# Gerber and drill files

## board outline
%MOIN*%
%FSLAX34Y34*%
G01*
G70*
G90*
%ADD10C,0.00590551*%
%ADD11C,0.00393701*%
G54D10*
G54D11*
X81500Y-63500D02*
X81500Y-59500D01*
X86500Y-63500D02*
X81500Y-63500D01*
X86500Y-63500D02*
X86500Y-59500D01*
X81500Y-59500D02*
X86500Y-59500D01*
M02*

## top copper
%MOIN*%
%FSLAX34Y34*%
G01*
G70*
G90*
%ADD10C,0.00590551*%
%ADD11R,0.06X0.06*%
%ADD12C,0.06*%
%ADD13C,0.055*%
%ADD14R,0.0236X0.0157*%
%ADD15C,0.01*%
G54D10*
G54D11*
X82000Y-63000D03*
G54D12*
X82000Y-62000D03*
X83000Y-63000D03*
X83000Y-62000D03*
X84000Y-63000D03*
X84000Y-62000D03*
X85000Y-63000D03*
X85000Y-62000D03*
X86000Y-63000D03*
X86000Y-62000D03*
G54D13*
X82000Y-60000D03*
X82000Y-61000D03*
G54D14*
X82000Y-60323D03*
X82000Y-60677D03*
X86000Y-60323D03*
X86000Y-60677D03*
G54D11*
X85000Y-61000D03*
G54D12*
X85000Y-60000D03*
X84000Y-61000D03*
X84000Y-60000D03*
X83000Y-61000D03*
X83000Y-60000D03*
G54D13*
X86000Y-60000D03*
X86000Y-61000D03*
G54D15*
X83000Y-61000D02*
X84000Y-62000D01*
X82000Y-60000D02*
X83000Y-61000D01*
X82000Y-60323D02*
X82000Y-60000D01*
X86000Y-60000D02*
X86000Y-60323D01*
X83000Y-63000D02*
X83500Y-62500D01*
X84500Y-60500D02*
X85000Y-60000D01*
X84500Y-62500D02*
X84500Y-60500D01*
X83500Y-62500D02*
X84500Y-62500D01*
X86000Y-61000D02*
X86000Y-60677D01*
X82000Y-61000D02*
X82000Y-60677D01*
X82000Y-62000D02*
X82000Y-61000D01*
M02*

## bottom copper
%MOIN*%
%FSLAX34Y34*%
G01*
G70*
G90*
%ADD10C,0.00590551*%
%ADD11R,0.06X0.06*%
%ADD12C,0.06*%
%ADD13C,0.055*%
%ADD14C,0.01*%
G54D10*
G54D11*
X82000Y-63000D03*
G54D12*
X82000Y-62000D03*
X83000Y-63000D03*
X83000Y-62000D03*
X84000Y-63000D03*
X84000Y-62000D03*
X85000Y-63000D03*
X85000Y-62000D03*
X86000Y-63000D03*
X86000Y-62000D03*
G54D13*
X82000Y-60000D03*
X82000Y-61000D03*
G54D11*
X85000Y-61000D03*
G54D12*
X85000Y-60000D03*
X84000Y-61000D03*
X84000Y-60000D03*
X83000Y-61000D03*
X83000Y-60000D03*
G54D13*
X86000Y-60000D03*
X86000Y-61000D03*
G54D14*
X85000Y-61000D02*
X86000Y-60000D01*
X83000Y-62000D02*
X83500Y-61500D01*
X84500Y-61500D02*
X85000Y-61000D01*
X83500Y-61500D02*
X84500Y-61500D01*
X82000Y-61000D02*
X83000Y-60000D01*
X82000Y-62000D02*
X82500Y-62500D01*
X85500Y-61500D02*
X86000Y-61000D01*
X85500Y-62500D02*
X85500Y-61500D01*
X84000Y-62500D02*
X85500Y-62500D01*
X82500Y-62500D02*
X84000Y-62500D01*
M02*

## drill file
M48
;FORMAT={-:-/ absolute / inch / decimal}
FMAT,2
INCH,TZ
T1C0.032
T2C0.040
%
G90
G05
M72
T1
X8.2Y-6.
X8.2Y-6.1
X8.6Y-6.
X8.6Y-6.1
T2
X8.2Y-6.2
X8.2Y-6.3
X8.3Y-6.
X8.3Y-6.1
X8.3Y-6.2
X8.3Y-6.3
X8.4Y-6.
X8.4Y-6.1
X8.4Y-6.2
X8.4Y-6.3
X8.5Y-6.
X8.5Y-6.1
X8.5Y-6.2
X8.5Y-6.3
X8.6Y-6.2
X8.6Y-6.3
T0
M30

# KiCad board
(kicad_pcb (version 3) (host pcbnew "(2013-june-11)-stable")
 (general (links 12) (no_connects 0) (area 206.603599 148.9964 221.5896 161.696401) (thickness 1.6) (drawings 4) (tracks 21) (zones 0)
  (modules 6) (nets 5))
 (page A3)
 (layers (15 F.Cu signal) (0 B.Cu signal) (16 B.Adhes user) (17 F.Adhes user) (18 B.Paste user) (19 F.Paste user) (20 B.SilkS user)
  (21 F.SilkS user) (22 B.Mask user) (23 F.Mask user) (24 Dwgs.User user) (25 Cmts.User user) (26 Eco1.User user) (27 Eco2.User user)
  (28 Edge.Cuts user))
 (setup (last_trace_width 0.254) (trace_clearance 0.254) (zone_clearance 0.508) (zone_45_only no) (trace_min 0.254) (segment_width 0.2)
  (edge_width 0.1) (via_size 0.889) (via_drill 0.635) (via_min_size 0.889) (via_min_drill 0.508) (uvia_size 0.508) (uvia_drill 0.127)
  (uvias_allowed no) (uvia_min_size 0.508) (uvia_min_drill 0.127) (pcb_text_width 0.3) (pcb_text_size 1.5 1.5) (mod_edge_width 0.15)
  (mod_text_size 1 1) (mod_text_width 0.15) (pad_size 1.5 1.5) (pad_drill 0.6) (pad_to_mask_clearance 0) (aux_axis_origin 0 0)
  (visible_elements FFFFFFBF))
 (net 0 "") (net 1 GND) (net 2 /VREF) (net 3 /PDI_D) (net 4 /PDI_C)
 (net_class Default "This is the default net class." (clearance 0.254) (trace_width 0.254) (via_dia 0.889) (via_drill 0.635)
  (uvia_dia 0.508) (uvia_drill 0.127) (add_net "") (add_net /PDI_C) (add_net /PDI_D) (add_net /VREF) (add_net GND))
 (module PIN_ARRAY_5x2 (layer F.Cu) (at 213.36 158.75)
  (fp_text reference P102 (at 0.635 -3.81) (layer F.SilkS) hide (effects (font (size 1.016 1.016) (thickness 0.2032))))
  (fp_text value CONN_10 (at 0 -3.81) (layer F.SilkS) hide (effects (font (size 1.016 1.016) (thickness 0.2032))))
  (pad 1 thru_hole rect (at -5.08 1.27) (size 1.524 1.524) (drill 1.016) (layers *.Cu *.Mask F.SilkS))
  (pad 2 thru_hole circle (at -5.08 -1.27) (size 1.524 1.524) (drill 1.016) (layers *.Cu *.Mask F.SilkS) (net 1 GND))
  (pad 3 thru_hole circle (at -2.54 1.27) (size 1.524 1.524) (drill 1.016) (layers *.Cu *.Mask F.SilkS) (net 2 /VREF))
  (pad 4 thru_hole circle (at -2.54 -1.27) (size 1.524 1.524) (drill 1.016) (layers *.Cu *.Mask F.SilkS) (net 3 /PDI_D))
  (pad 5 thru_hole circle (at 0 1.27) (size 1.524 1.524) (drill 1.016) (layers *.Cu *.Mask F.SilkS))
  (pad 6 thru_hole circle (at 0 -1.27) (size 1.524 1.524) (drill 1.016) (layers *.Cu *.Mask F.SilkS) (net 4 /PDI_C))
  (pad 7 thru_hole circle (at 2.54 1.27) (size 1.524 1.524) (drill 1.016) (layers *.Cu *.Mask F.SilkS))
  (pad 8 thru_hole circle (at 2.54 -1.27) (size 1.524 1.524) (drill 1.016) (layers *.Cu *.Mask F.SilkS))
  (pad 9 thru_hole circle (at 5.08 1.27) (size 1.524 1.524) (drill 1.016) (layers *.Cu *.Mask F.SilkS))
  (pad 10 thru_hole circle (at 5.08 -1.27) (size 1.524 1.524) (drill 1.016) (layers *.Cu *.Mask F.SilkS)))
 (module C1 (layer F.Cu) (at 208.28 153.67 270)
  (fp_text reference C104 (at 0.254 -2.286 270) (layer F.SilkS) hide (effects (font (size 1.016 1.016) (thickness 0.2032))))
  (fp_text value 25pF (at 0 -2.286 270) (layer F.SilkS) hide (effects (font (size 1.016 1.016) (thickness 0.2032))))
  (pad 1 thru_hole circle (at -1.27 0 270) (size 1.397 1.397) (drill 0.8128) (layers *.Cu *.Mask F.SilkS) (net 4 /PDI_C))
  (pad 2 thru_hole circle (at 1.27 0 270) (size 1.397 1.397) (drill 0.8128) (layers *.Cu *.Mask F.SilkS) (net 1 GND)))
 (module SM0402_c (layer F.Cu) (at 208.28 153.67 270)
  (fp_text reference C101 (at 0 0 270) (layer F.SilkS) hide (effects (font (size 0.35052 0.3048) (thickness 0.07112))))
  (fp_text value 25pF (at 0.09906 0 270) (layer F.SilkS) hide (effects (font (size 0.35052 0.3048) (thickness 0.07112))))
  (pad 1 smd rect (at -0.44958 0 270) (size 0.39878 0.59944) (layers F.Cu F.Paste F.Mask) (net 4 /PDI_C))
  (pad 2 smd rect (at 0.44958 0 270) (size 0.39878 0.59944) (layers F.Cu F.Paste F.Mask) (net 1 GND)))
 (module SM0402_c (layer F.Cu) (at 218.44 153.67 270)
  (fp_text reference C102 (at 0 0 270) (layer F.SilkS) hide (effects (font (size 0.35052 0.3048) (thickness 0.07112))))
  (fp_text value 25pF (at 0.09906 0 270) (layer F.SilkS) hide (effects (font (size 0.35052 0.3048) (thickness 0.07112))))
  (pad 1 smd rect (at -0.44958 0 270) (size 0.39878 0.59944) (layers F.Cu F.Paste F.Mask) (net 3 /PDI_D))
  (pad 2 smd rect (at 0.44958 0 270) (size 0.39878 0.59944) (layers F.Cu F.Paste F.Mask) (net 1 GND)))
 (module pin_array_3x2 (layer B.Cu) (at 213.36 153.67 180)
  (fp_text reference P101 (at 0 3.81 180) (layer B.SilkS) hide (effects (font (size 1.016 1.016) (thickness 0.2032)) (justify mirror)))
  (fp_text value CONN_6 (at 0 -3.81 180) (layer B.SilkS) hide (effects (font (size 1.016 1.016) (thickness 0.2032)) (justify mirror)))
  (pad 1 thru_hole rect (at -2.54 -1.27 180) (size 1.524 1.524) (drill 1.016) (layers *.Cu *.Mask B.SilkS) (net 3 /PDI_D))
  (pad 2 thru_hole circle (at -2.54 1.27 180) (size 1.524 1.524) (drill 1.016) (layers *.Cu *.Mask B.SilkS) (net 2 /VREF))
  (pad 3 thru_hole circle (at 0 -1.27 180) (size 1.524 1.524) (drill 1.016) (layers *.Cu *.Mask B.SilkS))
  (pad 4 thru_hole circle (at 0 1.27 180) (size 1.524 1.524) (drill 1.016) (layers *.Cu *.Mask B.SilkS))
  (pad 5 thru_hole circle (at 2.54 -1.27 180) (size 1.524 1.524) (drill 1.016) (layers *.Cu *.Mask B.SilkS) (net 4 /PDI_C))
  (pad 6 thru_hole circle (at 2.54 1.27 180) (size 1.524 1.524) (drill 1.016) (layers *.Cu *.Mask B.SilkS) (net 1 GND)))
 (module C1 (layer F.Cu) (at 218.44 153.67 270)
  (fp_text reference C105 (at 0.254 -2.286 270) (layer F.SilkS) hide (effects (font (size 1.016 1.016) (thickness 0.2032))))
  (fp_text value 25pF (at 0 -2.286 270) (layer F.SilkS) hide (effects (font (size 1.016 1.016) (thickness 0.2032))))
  (pad 1 thru_hole circle (at -1.27 0 270) (size 1.397 1.397) (drill 0.8128) (layers *.Cu *.Mask F.SilkS) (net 3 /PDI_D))
  (pad 2 thru_hole circle (at 1.27 0 270) (size 1.397 1.397) (drill 0.8128) (layers *.Cu *.Mask F.SilkS) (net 1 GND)))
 (gr_line (start 207.01 161.29) (end 207.01 151.13) (angle 90) (layer Edge.Cuts) (width 0.1))
 (gr_line (start 219.71 161.29) (end 207.01 161.29) (angle 90) (layer Edge.Cuts) (width 0.1))
 (gr_line (start 219.71 161.29) (end 219.71 151.13) (angle 90) (layer Edge.Cuts) (width 0.1))
 (gr_line (start 207.01 151.13) (end 219.71 151.13) (angle 90) (layer Edge.Cuts) (width 0.1))
 (segment (start 210.82 154.94) (end 213.36 157.48) (width 0.254) (layer F.Cu) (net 4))
 (segment (start 208.28 152.4) (end 210.82 154.94) (width 0.254) (layer F.Cu) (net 4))
 (segment (start 208.28 153.22042) (end 208.28 152.4) (width 0.254) (layer F.Cu) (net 4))
 (segment (start 215.9 154.94) (end 218.44 152.4) (width 0.254) (layer B.Cu) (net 3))
 (segment (start 210.82 157.48) (end 212.09 156.21) (width 0.254) (layer B.Cu) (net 3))
 (segment (start 214.63 156.21) (end 215.9 154.94) (width 0.254) (layer B.Cu) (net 3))
 (segment (start 212.09 156.21) (end 214.63 156.21) (width 0.254) (layer B.Cu) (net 3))
 (segment (start 218.44 152.4) (end 218.44 153.22042) (width 0.254) (layer F.Cu) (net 3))
 (segment (start 210.82 160.02) (end 212.09 158.75) (width 0.254) (layer F.Cu) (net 2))
 (segment (start 214.63 153.67) (end 215.9 152.4) (width 0.254) (layer F.Cu) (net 2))
 (segment (start 214.63 158.75) (end 214.63 153.67) (width 0.254) (layer F.Cu) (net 2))
 (segment (start 212.09 158.75) (end 214.63 158.75) (width 0.254) (layer F.Cu) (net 2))
 (segment (start 208.28 154.94) (end 210.82 152.4) (width 0.254) (layer B.Cu) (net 1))
 (segment (start 208.28 157.48) (end 209.55 158.75) (width 0.254) (layer B.Cu) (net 1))
 (segment (start 217.17 156.21) (end 218.44 154.94) (width 0.254) (layer B.Cu) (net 1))
 (segment (start 217.17 158.75) (end 217.17 156.21) (width 0.254) (layer B.Cu) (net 1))
 (segment (start 213.36 158.75) (end 217.17 158.75) (width 0.254) (layer B.Cu) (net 1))
 (segment (start 209.55 158.75) (end 213.36 158.75) (width 0.254) (layer B.Cu) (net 1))
 (segment (start 218.44 154.94) (end 218.44 154.11958) (width 0.254) (layer F.Cu) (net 1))
 (segment (start 208.28 154.94) (end 208.28 154.11958) (width 0.254) (layer F.Cu) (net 1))
 (segment (start 208.28 157.48) (end 208.28 154.94) (width 0.254) (layer F.Cu) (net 1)))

